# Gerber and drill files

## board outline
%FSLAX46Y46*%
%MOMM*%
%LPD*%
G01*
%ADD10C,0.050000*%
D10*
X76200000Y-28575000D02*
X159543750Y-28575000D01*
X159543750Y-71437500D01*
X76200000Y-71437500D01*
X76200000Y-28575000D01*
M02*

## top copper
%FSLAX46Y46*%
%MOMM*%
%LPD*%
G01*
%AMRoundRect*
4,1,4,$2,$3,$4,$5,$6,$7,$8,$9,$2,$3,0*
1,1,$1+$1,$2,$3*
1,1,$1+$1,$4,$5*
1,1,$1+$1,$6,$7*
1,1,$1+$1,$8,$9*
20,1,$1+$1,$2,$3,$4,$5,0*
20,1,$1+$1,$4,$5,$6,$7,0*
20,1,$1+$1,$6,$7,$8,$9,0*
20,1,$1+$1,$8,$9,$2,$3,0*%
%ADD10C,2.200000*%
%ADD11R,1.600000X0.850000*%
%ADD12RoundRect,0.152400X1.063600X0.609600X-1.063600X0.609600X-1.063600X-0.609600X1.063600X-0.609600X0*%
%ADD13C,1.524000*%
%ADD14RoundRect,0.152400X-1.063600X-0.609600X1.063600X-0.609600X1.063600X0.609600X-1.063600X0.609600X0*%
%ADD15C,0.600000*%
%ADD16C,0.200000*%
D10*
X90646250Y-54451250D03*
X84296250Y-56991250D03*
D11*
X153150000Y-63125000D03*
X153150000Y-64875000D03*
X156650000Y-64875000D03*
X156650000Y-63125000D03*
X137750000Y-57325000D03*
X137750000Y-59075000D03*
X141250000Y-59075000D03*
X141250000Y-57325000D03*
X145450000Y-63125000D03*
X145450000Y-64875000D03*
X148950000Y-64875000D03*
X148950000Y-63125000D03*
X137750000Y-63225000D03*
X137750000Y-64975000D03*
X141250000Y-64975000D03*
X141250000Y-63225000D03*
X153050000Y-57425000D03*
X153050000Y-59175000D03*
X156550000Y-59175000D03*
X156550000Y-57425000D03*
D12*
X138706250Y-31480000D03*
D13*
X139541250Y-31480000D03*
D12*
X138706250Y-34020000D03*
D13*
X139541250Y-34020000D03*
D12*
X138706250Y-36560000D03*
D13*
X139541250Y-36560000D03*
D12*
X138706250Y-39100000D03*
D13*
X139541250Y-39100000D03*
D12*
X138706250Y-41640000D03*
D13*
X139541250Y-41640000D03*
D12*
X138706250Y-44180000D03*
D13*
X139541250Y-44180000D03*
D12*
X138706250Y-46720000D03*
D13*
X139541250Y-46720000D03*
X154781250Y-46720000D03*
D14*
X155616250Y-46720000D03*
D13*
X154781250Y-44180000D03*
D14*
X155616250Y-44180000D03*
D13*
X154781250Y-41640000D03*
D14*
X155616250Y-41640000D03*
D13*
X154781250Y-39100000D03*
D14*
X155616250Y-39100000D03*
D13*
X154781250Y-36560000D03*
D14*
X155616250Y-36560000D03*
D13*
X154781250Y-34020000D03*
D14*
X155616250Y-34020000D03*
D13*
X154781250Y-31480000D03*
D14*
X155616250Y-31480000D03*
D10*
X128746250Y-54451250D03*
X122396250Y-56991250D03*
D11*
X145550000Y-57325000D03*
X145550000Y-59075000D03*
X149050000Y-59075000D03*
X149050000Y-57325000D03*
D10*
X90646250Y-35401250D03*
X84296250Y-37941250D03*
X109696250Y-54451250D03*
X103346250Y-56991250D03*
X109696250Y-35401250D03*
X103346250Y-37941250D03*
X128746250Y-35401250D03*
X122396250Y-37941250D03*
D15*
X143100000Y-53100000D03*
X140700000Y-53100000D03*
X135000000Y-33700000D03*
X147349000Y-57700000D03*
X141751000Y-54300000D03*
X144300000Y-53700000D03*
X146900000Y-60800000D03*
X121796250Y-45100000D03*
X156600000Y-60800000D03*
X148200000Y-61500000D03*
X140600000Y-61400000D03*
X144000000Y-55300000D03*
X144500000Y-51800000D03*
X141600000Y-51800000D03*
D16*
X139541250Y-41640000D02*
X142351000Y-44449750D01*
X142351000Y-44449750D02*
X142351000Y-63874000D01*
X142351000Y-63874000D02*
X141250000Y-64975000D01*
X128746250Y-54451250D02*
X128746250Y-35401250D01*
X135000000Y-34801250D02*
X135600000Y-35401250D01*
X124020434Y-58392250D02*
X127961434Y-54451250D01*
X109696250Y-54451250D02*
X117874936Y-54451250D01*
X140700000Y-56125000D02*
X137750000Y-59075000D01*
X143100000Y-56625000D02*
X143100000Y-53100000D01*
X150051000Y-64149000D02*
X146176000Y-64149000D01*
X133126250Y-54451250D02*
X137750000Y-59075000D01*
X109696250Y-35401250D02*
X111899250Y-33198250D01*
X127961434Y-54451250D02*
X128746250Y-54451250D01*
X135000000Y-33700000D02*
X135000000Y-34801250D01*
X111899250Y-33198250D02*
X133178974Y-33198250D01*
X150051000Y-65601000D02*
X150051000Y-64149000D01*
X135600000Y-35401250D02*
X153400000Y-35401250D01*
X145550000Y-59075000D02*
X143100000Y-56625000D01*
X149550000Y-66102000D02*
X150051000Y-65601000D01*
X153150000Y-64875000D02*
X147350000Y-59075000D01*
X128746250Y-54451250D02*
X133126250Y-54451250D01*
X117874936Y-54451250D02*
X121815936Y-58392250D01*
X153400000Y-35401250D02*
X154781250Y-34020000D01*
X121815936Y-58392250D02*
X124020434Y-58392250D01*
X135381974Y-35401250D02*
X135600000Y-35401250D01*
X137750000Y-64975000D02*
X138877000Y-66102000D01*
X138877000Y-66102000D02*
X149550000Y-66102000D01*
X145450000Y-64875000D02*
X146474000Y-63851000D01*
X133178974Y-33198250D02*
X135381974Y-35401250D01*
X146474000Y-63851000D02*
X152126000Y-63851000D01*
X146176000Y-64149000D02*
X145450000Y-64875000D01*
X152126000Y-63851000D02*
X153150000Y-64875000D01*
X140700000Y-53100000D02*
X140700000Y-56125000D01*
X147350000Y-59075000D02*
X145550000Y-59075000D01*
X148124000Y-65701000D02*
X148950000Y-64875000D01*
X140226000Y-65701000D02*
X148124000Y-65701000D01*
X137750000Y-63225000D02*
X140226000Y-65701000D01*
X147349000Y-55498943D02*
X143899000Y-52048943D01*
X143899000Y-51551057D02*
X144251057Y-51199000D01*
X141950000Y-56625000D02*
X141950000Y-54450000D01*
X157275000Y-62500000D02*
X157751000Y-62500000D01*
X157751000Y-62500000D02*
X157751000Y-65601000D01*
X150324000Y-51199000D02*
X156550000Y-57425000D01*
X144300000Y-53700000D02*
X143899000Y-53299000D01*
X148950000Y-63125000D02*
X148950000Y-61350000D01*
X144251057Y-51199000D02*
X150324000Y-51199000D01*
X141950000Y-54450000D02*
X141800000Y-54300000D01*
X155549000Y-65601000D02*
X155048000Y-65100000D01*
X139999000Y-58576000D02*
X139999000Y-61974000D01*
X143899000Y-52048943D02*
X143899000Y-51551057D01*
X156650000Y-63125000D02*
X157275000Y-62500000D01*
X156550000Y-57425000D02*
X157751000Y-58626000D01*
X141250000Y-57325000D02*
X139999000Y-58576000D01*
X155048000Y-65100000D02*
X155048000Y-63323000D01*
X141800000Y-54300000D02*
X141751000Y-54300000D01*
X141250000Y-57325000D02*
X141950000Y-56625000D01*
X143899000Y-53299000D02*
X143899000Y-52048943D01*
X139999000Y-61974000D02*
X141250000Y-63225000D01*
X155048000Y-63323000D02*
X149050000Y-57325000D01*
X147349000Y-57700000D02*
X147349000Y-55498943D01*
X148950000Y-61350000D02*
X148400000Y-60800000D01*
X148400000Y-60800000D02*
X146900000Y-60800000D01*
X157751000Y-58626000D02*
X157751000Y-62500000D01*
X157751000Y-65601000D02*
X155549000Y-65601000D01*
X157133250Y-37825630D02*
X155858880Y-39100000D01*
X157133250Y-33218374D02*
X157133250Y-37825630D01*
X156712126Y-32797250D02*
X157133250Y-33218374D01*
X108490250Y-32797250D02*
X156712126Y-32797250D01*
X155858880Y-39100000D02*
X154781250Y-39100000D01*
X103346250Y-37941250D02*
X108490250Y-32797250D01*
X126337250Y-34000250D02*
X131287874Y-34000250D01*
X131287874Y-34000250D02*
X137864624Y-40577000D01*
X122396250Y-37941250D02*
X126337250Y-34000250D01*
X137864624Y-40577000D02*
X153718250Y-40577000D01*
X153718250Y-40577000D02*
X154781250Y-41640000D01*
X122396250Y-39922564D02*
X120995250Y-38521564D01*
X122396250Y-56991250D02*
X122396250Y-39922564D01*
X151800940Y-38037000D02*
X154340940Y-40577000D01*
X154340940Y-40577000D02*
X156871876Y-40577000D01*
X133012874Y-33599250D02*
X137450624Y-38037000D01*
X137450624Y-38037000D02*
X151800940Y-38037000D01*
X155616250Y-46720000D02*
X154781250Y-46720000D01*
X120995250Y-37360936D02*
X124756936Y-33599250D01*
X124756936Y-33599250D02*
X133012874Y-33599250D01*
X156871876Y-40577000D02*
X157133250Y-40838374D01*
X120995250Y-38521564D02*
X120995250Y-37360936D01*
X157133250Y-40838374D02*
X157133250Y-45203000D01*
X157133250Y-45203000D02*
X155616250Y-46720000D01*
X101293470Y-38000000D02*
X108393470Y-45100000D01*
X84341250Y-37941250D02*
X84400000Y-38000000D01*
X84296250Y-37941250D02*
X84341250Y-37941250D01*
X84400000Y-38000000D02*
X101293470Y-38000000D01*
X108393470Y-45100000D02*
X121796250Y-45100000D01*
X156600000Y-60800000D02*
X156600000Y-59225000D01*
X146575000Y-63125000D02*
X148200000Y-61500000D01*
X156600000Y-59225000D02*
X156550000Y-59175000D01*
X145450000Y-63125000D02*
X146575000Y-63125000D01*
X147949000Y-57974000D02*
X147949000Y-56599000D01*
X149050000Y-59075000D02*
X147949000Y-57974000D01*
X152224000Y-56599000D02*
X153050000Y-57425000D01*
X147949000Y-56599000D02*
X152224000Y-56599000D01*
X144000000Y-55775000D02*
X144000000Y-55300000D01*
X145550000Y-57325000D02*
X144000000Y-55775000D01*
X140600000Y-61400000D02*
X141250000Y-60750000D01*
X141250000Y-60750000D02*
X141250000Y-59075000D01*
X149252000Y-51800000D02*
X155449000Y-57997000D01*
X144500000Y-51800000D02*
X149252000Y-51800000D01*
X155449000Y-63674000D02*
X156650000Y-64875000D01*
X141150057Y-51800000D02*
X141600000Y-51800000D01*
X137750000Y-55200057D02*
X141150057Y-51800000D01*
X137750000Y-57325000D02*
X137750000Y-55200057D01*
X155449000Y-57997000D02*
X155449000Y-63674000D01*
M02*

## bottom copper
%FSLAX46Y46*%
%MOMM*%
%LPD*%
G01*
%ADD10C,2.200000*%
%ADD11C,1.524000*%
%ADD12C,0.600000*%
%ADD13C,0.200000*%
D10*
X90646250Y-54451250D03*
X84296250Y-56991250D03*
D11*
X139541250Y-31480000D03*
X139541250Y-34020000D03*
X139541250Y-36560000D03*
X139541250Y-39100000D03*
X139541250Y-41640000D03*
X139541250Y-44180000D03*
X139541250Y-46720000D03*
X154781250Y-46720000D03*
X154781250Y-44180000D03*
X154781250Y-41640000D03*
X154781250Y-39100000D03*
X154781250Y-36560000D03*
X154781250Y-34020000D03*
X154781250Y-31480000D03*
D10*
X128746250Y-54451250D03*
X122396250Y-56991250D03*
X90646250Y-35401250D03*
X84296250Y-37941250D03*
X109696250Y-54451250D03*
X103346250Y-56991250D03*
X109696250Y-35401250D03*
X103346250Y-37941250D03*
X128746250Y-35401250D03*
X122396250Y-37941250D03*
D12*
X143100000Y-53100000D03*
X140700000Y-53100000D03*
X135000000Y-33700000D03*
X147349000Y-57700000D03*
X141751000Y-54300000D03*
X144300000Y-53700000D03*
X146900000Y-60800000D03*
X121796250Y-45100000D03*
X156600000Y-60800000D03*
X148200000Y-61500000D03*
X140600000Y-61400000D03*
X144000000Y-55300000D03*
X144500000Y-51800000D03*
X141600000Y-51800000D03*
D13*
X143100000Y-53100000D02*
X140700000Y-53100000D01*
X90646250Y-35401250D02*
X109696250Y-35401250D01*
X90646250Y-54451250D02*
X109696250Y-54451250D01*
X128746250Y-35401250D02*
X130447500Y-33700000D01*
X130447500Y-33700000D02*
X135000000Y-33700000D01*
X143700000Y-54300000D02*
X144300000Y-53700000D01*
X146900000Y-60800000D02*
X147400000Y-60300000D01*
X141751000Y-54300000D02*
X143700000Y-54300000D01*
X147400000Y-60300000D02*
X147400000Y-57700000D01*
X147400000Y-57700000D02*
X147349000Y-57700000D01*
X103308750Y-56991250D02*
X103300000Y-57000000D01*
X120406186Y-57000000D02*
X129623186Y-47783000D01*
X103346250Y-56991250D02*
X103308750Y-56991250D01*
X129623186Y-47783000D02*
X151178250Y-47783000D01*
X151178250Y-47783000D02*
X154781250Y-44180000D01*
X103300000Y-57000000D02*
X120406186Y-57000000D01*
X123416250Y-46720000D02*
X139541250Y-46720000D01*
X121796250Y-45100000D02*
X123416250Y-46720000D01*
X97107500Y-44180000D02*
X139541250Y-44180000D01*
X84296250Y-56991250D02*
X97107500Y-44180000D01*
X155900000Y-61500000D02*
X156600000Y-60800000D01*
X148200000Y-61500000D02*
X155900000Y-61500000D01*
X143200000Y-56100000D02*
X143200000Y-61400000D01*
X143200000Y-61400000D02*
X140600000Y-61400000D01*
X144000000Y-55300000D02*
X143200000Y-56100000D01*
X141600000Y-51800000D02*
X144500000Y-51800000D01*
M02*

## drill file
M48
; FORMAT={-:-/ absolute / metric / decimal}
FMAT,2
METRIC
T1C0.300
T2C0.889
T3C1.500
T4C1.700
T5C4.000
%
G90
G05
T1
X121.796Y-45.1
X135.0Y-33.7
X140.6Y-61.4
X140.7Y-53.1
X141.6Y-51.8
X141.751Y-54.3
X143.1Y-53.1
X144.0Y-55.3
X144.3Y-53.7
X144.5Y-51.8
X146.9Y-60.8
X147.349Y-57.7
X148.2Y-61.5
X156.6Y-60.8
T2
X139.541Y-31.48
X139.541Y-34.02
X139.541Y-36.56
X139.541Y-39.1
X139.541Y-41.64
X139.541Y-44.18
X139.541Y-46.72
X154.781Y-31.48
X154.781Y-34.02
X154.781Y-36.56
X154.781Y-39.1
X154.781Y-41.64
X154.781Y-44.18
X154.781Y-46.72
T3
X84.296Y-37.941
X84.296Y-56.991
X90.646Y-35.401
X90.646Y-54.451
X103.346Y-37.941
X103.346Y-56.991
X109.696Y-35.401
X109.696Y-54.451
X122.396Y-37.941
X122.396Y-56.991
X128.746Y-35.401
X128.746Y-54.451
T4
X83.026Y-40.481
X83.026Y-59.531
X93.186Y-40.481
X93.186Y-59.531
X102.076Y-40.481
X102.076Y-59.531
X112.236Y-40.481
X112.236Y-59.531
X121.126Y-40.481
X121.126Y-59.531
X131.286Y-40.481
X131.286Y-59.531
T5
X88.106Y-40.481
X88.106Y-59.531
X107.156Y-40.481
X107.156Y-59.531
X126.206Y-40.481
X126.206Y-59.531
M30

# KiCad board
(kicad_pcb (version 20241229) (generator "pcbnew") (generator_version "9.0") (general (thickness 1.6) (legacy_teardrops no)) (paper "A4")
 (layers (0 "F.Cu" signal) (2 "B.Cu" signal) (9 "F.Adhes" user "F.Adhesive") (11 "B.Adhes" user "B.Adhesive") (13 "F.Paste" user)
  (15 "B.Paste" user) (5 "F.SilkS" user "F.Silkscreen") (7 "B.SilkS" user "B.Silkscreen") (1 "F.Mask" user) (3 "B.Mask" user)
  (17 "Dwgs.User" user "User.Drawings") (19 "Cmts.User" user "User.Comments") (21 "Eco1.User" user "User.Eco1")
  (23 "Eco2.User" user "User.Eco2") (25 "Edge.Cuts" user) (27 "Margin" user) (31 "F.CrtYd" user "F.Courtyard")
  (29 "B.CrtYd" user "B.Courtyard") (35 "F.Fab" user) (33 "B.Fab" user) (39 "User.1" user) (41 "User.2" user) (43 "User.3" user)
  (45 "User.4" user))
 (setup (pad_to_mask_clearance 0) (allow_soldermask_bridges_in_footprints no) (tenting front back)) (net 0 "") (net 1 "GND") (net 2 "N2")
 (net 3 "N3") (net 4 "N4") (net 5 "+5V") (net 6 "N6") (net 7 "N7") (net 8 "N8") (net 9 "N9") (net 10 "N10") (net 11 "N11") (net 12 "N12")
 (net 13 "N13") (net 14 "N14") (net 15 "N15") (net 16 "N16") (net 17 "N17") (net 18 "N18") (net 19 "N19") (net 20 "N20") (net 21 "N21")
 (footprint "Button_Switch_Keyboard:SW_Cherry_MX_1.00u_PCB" (layer "F.Cu") (at 90.64625 54.45125)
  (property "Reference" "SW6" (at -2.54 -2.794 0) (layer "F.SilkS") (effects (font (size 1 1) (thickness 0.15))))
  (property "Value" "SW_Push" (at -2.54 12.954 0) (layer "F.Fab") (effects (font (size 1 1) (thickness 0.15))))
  (pad "" np_thru_hole circle (at -7.62 5.08) (size 1.7 1.7) (drill 1.7) (layers "*.Cu" "*.Mask"))
  (pad "" np_thru_hole circle (at -2.54 5.08) (size 4 4) (drill 4) (layers "*.Cu" "*.Mask"))
  (pad "" np_thru_hole circle (at 2.54 5.08) (size 1.7 1.7) (drill 1.7) (layers "*.Cu" "*.Mask"))
  (pad "1" thru_hole circle (at 0 0) (size 2.2 2.2) (drill 1.5) (layers "*.Cu" "*.Mask") (remove_unused_layers no) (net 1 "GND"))
  (pad "2" thru_hole circle (at -6.35 2.54) (size 2.2 2.2) (drill 1.5) (layers "*.Cu" "*.Mask") (remove_unused_layers no) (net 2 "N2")))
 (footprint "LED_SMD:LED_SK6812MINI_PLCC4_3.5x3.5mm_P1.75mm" (layer "F.Cu") (at 154.9 64)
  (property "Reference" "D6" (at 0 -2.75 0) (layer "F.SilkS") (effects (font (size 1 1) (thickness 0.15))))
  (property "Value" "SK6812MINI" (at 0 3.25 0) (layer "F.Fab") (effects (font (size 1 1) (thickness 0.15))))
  (pad "1" smd rect (at -1.75 -0.875) (size 1.6 0.85) (layers "F.Cu" "F.Mask" "F.Paste") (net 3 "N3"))
  (pad "2" smd rect (at -1.75 0.875) (size 1.6 0.85) (layers "F.Cu" "F.Mask" "F.Paste") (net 1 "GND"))
  (pad "3" smd rect (at 1.75 0.875) (size 1.6 0.85) (layers "F.Cu" "F.Mask" "F.Paste") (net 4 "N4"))
  (pad "4" smd rect (at 1.75 -0.875) (size 1.6 0.85) (layers "F.Cu" "F.Mask" "F.Paste") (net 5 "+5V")))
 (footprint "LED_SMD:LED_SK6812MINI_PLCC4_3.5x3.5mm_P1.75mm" (layer "F.Cu") (at 139.5 58.2)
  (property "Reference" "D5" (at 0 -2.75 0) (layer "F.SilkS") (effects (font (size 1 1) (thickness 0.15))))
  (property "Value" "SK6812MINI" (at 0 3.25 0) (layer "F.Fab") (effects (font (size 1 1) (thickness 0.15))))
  (pad "1" smd rect (at -1.75 -0.875) (size 1.6 0.85) (layers "F.Cu" "F.Mask" "F.Paste") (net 4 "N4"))
  (pad "2" smd rect (at -1.75 0.875) (size 1.6 0.85) (layers "F.Cu" "F.Mask" "F.Paste") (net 1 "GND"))
  (pad "3" smd rect (at 1.75 0.875) (size 1.6 0.85) (layers "F.Cu" "F.Mask" "F.Paste") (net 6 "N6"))
  (pad "4" smd rect (at 1.75 -0.875) (size 1.6 0.85) (layers "F.Cu" "F.Mask" "F.Paste") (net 5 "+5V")))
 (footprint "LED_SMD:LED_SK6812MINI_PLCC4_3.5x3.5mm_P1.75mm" (layer "F.Cu") (at 147.2 64)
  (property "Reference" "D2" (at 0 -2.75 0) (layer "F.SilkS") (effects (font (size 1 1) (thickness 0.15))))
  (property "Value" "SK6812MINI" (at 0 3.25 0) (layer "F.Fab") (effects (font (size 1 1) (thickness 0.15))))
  (pad "1" smd rect (at -1.75 -0.875) (size 1.6 0.85) (layers "F.Cu" "F.Mask" "F.Paste") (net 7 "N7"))
  (pad "2" smd rect (at -1.75 0.875) (size 1.6 0.85) (layers "F.Cu" "F.Mask" "F.Paste") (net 1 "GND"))
  (pad "3" smd rect (at 1.75 0.875) (size 1.6 0.85) (layers "F.Cu" "F.Mask" "F.Paste") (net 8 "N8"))
  (pad "4" smd rect (at 1.75 -0.875) (size 1.6 0.85) (layers "F.Cu" "F.Mask" "F.Paste") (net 5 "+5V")))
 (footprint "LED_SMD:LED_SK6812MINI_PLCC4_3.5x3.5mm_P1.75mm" (layer "F.Cu") (at 139.5 64.1)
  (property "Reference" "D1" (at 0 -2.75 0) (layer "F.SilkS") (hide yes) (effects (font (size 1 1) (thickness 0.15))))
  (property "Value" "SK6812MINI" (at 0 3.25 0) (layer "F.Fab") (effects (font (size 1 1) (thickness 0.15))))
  (pad "1" smd rect (at -1.75 -0.875) (size 1.6 0.85) (layers "F.Cu" "F.Mask" "F.Paste") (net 8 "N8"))
  (pad "2" smd rect (at -1.75 0.875) (size 1.6 0.85) (layers "F.Cu" "F.Mask" "F.Paste") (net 1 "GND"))
  (pad "3" smd rect (at 1.75 0.875) (size 1.6 0.85) (layers "F.Cu" "F.Mask" "F.Paste") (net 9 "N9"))
  (pad "4" smd rect (at 1.75 -0.875) (size 1.6 0.85) (layers "F.Cu" "F.Mask" "F.Paste") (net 5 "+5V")))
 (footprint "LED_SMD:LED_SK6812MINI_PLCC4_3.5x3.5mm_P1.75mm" (layer "F.Cu") (at 154.8 58.3)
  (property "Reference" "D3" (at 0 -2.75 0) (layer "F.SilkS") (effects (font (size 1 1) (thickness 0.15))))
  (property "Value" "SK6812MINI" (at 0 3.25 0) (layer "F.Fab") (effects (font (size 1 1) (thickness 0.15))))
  (pad "1" smd rect (at -1.75 -0.875) (size 1.6 0.85) (layers "F.Cu" "F.Mask" "F.Paste") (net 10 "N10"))
  (pad "2" smd rect (at -1.75 0.875) (size 1.6 0.85) (layers "F.Cu" "F.Mask" "F.Paste") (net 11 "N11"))
  (pad "3" smd rect (at 1.75 0.875) (size 1.6 0.85) (layers "F.Cu" "F.Mask" "F.Paste") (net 7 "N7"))
  (pad "4" smd rect (at 1.75 -0.875) (size 1.6 0.85) (layers "F.Cu" "F.Mask" "F.Paste") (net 5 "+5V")))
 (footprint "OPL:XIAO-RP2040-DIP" (layer "F.Cu") (at 147.16125 39.1)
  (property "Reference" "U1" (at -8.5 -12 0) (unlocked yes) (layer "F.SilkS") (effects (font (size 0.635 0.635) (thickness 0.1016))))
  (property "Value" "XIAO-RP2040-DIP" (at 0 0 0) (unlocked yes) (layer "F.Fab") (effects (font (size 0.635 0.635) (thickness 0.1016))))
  (pad "1" smd roundrect (at -8.455 -7.62 180) (size 2.432 1.524) (layers "F.Cu" "F.Mask") (roundrect_rratio 0.1) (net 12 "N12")
   (thermal_bridge_angle 45))
  (pad "1" thru_hole circle (at -7.62 -7.62 180) (size 1.524 1.524) (drill 0.889) (layers "*.Cu" "*.Mask") (remove_unused_layers no)
   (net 12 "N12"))
  (pad "2" smd roundrect (at -8.455 -5.08 180) (size 2.432 1.524) (layers "F.Cu" "F.Mask") (roundrect_rratio 0.1) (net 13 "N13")
   (thermal_bridge_angle 45))
  (pad "2" thru_hole circle (at -7.62 -5.08 180) (size 1.524 1.524) (drill 0.889) (layers "*.Cu" "*.Mask") (remove_unused_layers no)
   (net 13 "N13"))
  (pad "3" smd roundrect (at -8.455 -2.54 180) (size 2.432 1.524) (layers "F.Cu" "F.Mask") (roundrect_rratio 0.1) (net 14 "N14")
   (thermal_bridge_angle 45))
  (pad "3" thru_hole circle (at -7.62 -2.54 180) (size 1.524 1.524) (drill 0.889) (layers "*.Cu" "*.Mask") (remove_unused_layers no)
   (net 14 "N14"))
  (pad "4" smd roundrect (at -8.455 0 180) (size 2.432 1.524) (layers "F.Cu" "F.Mask") (roundrect_rratio 0.1) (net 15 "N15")
   (thermal_bridge_angle 45))
  (pad "4" thru_hole circle (at -7.62 0 180) (size 1.524 1.524) (drill 0.889) (layers "*.Cu" "*.Mask") (remove_unused_layers no)
   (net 15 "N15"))
  (pad "5" smd roundrect (at -8.455 2.54 180) (size 2.432 1.524) (layers "F.Cu" "F.Mask") (roundrect_rratio 0.1) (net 9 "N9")
   (thermal_bridge_angle 45))
  (pad "5" thru_hole circle (at -7.62 2.54 180) (size 1.524 1.524) (drill 0.889) (layers "*.Cu" "*.Mask") (remove_unused_layers no)
   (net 9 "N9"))
  (pad "6" smd roundrect (at -8.455 5.08 180) (size 2.432 1.524) (layers "F.Cu" "F.Mask") (roundrect_rratio 0.1) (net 2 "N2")
   (thermal_bridge_angle 45))
  (pad "6" thru_hole circle (at -7.62 5.08 180) (size 1.524 1.524) (drill 0.889) (layers "*.Cu" "*.Mask") (remove_unused_layers no)
   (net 2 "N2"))
  (pad "7" smd roundrect (at -8.455 7.62 180) (size 2.432 1.524) (layers "F.Cu" "F.Mask") (roundrect_rratio 0.1) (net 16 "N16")
   (thermal_bridge_angle 45))
  (pad "7" thru_hole circle (at -7.62 7.62 180) (size 1.524 1.524) (drill 0.889) (layers "*.Cu" "*.Mask") (remove_unused_layers no)
   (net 16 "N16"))
  (pad "8" thru_hole circle (at 7.62 7.62) (size 1.524 1.524) (drill 0.889) (layers "*.Cu" "*.Mask") (remove_unused_layers no)
   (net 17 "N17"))
  (pad "8" smd roundrect (at 8.455 7.62) (size 2.432 1.524) (layers "F.Cu" "F.Mask") (roundrect_rratio 0.1) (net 17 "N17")
   (thermal_bridge_angle 45))
  (pad "9" thru_hole circle (at 7.62 5.08) (size 1.524 1.524) (drill 0.889) (layers "*.Cu" "*.Mask") (remove_unused_layers no)
   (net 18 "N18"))
  (pad "9" smd roundrect (at 8.455 5.08) (size 2.432 1.524) (layers "F.Cu" "F.Mask") (roundrect_rratio 0.1) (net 18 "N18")
   (thermal_bridge_angle 45))
  (pad "10" thru_hole circle (at 7.62 2.54) (size 1.524 1.524) (drill 0.889) (layers "*.Cu" "*.Mask") (remove_unused_layers no)
   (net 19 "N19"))
  (pad "10" smd roundrect (at 8.455 2.54) (size 2.432 1.524) (layers "F.Cu" "F.Mask") (roundrect_rratio 0.1) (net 19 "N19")
   (thermal_bridge_angle 45))
  (pad "11" thru_hole circle (at 7.62 0) (size 1.524 1.524) (drill 0.889) (layers "*.Cu" "*.Mask") (remove_unused_layers no) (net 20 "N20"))
  (pad "11" smd roundrect (at 8.455 0) (size 2.432 1.524) (layers "F.Cu" "F.Mask") (roundrect_rratio 0.1) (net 20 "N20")
   (thermal_bridge_angle 45))
  (pad "12" thru_hole circle (at 7.62 -2.54) (size 1.524 1.524) (drill 0.889) (layers "*.Cu" "*.Mask") (remove_unused_layers no)
   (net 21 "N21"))
  (pad "12" smd roundrect (at 8.455 -2.54) (size 2.432 1.524) (layers "F.Cu" "F.Mask") (roundrect_rratio 0.1) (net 21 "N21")
   (thermal_bridge_angle 45))
  (pad "13" thru_hole circle (at 7.62 -5.08) (size 1.524 1.524) (drill 0.889) (layers "*.Cu" "*.Mask") (remove_unused_layers no)
   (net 1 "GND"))
  (pad "13" smd roundrect (at 8.455 -5.08) (size 2.432 1.524) (layers "F.Cu" "F.Mask") (roundrect_rratio 0.1) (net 1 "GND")
   (thermal_bridge_angle 45))
  (pad "14" thru_hole circle (at 7.62 -7.62) (size 1.524 1.524) (drill 0.889) (layers "*.Cu" "*.Mask") (remove_unused_layers no)
   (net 5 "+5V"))
  (pad "14" smd roundrect (at 8.455 -7.62) (size 2.432 1.524) (layers "F.Cu" "F.Mask") (roundrect_rratio 0.1) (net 5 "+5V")
   (thermal_bridge_angle 45)))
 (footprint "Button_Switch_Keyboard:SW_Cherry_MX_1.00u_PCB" (layer "F.Cu") (at 128.74625 54.45125)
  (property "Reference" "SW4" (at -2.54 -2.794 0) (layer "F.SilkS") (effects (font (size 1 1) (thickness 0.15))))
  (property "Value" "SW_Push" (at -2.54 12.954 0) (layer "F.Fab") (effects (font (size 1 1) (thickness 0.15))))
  (pad "" np_thru_hole circle (at -7.62 5.08) (size 1.7 1.7) (drill 1.7) (layers "*.Cu" "*.Mask"))
  (pad "" np_thru_hole circle (at -2.54 5.08) (size 4 4) (drill 4) (layers "*.Cu" "*.Mask"))
  (pad "" np_thru_hole circle (at 2.54 5.08) (size 1.7 1.7) (drill 1.7) (layers "*.Cu" "*.Mask"))
  (pad "1" thru_hole circle (at 0 0) (size 2.2 2.2) (drill 1.5) (layers "*.Cu" "*.Mask") (remove_unused_layers no) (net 1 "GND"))
  (pad "2" thru_hole circle (at -6.35 2.54) (size 2.2 2.2) (drill 1.5) (layers "*.Cu" "*.Mask") (remove_unused_layers no) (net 17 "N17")))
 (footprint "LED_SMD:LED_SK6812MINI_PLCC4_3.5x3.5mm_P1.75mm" (layer "F.Cu") (at 147.3 58.2)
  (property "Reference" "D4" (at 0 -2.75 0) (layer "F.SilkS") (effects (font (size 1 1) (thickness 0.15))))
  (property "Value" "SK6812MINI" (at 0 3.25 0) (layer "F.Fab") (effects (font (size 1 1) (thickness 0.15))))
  (pad "1" smd rect (at -1.75 -0.875) (size 1.6 0.85) (layers "F.Cu" "F.Mask" "F.Paste") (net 6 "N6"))
  (pad "2" smd rect (at -1.75 0.875) (size 1.6 0.85) (layers "F.Cu" "F.Mask" "F.Paste") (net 1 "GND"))
  (pad "3" smd rect (at 1.75 0.875) (size 1.6 0.85) (layers "F.Cu" "F.Mask" "F.Paste") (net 10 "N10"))
  (pad "4" smd rect (at 1.75 -0.875) (size 1.6 0.85) (layers "F.Cu" "F.Mask" "F.Paste") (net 5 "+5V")))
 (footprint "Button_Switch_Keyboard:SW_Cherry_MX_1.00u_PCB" (layer "F.Cu") (at 90.64625 35.40125)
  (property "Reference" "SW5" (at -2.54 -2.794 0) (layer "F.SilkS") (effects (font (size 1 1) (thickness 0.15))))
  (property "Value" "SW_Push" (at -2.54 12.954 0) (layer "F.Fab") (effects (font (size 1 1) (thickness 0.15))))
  (pad "" np_thru_hole circle (at -7.62 5.08) (size 1.7 1.7) (drill 1.7) (layers "*.Cu" "*.Mask"))
  (pad "" np_thru_hole circle (at -2.54 5.08) (size 4 4) (drill 4) (layers "*.Cu" "*.Mask"))
  (pad "" np_thru_hole circle (at 2.54 5.08) (size 1.7 1.7) (drill 1.7) (layers "*.Cu" "*.Mask"))
  (pad "1" thru_hole circle (at 0 0) (size 2.2 2.2) (drill 1.5) (layers "*.Cu" "*.Mask") (remove_unused_layers no) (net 1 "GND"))
  (pad "2" thru_hole circle (at -6.35 2.54) (size 2.2 2.2) (drill 1.5) (layers "*.Cu" "*.Mask") (remove_unused_layers no) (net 16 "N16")))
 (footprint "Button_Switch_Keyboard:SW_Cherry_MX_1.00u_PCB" (layer "F.Cu") (at 109.69625 54.45125)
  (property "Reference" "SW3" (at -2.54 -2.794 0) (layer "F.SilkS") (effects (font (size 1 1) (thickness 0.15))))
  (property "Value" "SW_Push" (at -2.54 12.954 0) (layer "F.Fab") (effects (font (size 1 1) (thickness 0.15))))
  (pad "" np_thru_hole circle (at -7.62 5.08) (size 1.7 1.7) (drill 1.7) (layers "*.Cu" "*.Mask"))
  (pad "" np_thru_hole circle (at -2.54 5.08) (size 4 4) (drill 4) (layers "*.Cu" "*.Mask"))
  (pad "" np_thru_hole circle (at 2.54 5.08) (size 1.7 1.7) (drill 1.7) (layers "*.Cu" "*.Mask"))
  (pad "1" thru_hole circle (at 0 0) (size 2.2 2.2) (drill 1.5) (layers "*.Cu" "*.Mask") (remove_unused_layers no) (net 1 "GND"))
  (pad "2" thru_hole circle (at -6.35 2.54) (size 2.2 2.2) (drill 1.5) (layers "*.Cu" "*.Mask") (remove_unused_layers no) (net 18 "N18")))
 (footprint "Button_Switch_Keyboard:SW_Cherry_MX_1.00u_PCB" (layer "F.Cu") (at 109.69625 35.40125)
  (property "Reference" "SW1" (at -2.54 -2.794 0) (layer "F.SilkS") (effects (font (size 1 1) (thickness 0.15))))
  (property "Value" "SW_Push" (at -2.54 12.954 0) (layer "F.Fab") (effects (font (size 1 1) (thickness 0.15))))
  (pad "" np_thru_hole circle (at -7.62 5.08) (size 1.7 1.7) (drill 1.7) (layers "*.Cu" "*.Mask"))
  (pad "" np_thru_hole circle (at -2.54 5.08) (size 4 4) (drill 4) (layers "*.Cu" "*.Mask"))
  (pad "" np_thru_hole circle (at 2.54 5.08) (size 1.7 1.7) (drill 1.7) (layers "*.Cu" "*.Mask"))
  (pad "1" thru_hole circle (at 0 0) (size 2.2 2.2) (drill 1.5) (layers "*.Cu" "*.Mask") (remove_unused_layers no) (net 1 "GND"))
  (pad "2" thru_hole circle (at -6.35 2.54) (size 2.2 2.2) (drill 1.5) (layers "*.Cu" "*.Mask") (remove_unused_layers no) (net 20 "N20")))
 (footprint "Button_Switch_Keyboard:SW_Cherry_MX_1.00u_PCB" (layer "F.Cu") (at 128.74625 35.40125)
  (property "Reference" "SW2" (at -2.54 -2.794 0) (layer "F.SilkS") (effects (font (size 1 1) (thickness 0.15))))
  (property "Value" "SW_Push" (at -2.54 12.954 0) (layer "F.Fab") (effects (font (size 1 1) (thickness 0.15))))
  (pad "" np_thru_hole circle (at -7.62 5.08) (size 1.7 1.7) (drill 1.7) (layers "*.Cu" "*.Mask"))
  (pad "" np_thru_hole circle (at -2.54 5.08) (size 4 4) (drill 4) (layers "*.Cu" "*.Mask"))
  (pad "" np_thru_hole circle (at 2.54 5.08) (size 1.7 1.7) (drill 1.7) (layers "*.Cu" "*.Mask"))
  (pad "1" thru_hole circle (at 0 0) (size 2.2 2.2) (drill 1.5) (layers "*.Cu" "*.Mask") (remove_unused_layers no) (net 1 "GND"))
  (pad "2" thru_hole circle (at -6.35 2.54) (size 2.2 2.2) (drill 1.5) (layers "*.Cu" "*.Mask") (remove_unused_layers no) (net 19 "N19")))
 (gr_rect (start 76.2 28.575) (end 159.54375 71.4375) (stroke (width 0.05) (type default)) (fill no) (layer "Edge.Cuts"))
 (segment (start 139.54125 41.64) (end 142.351 44.44975) (width 0.2) (layer "F.Cu") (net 9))
 (segment (start 142.351 44.44975) (end 142.351 63.874) (width 0.2) (layer "F.Cu") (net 9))
 (segment (start 142.351 63.874) (end 141.25 64.975) (width 0.2) (layer "F.Cu") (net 9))
 (segment (start 128.74625 54.45125) (end 128.74625 35.40125) (width 0.2) (layer "F.Cu") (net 1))
 (segment (start 135 34.80125) (end 135.6 35.40125) (width 0.2) (layer "F.Cu") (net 1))
 (segment (start 124.020434 58.39225) (end 127.961434 54.45125) (width 0.2) (layer "F.Cu") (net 1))
 (segment (start 109.69625 54.45125) (end 117.874936 54.45125) (width 0.2) (layer "F.Cu") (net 1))
 (segment (start 140.7 56.125) (end 137.75 59.075) (width 0.2) (layer "F.Cu") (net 1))
 (segment (start 143.1 56.625) (end 143.1 53.1) (width 0.2) (layer "F.Cu") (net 1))
 (segment (start 150.051 64.149) (end 146.176 64.149) (width 0.2) (layer "F.Cu") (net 1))
 (segment (start 133.12625 54.45125) (end 137.75 59.075) (width 0.2) (layer "F.Cu") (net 1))
 (segment (start 109.69625 35.40125) (end 111.89925 33.19825) (width 0.2) (layer "F.Cu") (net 1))
 (segment (start 127.961434 54.45125) (end 128.74625 54.45125) (width 0.2) (layer "F.Cu") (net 1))
 (segment (start 135 33.7) (end 135 34.80125) (width 0.2) (layer "F.Cu") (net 1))
 (segment (start 111.89925 33.19825) (end 133.178974 33.19825) (width 0.2) (layer "F.Cu") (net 1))
 (segment (start 150.051 65.601) (end 150.051 64.149) (width 0.2) (layer "F.Cu") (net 1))
 (segment (start 135.6 35.40125) (end 153.4 35.40125) (width 0.2) (layer "F.Cu") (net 1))
 (segment (start 145.55 59.075) (end 143.1 56.625) (width 0.2) (layer "F.Cu") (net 1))
 (segment (start 149.55 66.102) (end 150.051 65.601) (width 0.2) (layer "F.Cu") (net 1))
 (segment (start 153.15 64.875) (end 147.35 59.075) (width 0.2) (layer "F.Cu") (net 1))
 (segment (start 128.74625 54.45125) (end 133.12625 54.45125) (width 0.2) (layer "F.Cu") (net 1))
 (segment (start 117.874936 54.45125) (end 121.815936 58.39225) (width 0.2) (layer "F.Cu") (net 1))
 (segment (start 153.4 35.40125) (end 154.78125 34.02) (width 0.2) (layer "F.Cu") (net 1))
 (segment (start 121.815936 58.39225) (end 124.020434 58.39225) (width 0.2) (layer "F.Cu") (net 1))
 (segment (start 135.381974 35.40125) (end 135.6 35.40125) (width 0.2) (layer "F.Cu") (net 1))
 (segment (start 137.75 64.975) (end 138.877 66.102) (width 0.2) (layer "F.Cu") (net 1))
 (segment (start 138.877 66.102) (end 149.55 66.102) (width 0.2) (layer "F.Cu") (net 1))
 (segment (start 145.45 64.875) (end 146.474 63.851) (width 0.2) (layer "F.Cu") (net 1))
 (segment (start 133.178974 33.19825) (end 135.381974 35.40125) (width 0.2) (layer "F.Cu") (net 1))
 (segment (start 146.474 63.851) (end 152.126 63.851) (width 0.2) (layer "F.Cu") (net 1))
 (segment (start 146.176 64.149) (end 145.45 64.875) (width 0.2) (layer "F.Cu") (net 1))
 (segment (start 152.126 63.851) (end 153.15 64.875) (width 0.2) (layer "F.Cu") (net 1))
 (segment (start 140.7 53.1) (end 140.7 56.125) (width 0.2) (layer "F.Cu") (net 1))
 (segment (start 147.35 59.075) (end 145.55 59.075) (width 0.2) (layer "F.Cu") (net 1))
 (via (at 143.1 53.1) (size 0.6) (drill 0.3) (layers "F.Cu" "B.Cu") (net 1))
 (via (at 140.7 53.1) (size 0.6) (drill 0.3) (layers "F.Cu" "B.Cu") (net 1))
 (via (at 135 33.7) (size 0.6) (drill 0.3) (layers "F.Cu" "B.Cu") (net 1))
 (segment (start 143.1 53.1) (end 140.7 53.1) (width 0.2) (layer "B.Cu") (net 1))
 (segment (start 90.64625 35.40125) (end 109.69625 35.40125) (width 0.2) (layer "B.Cu") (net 1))
 (segment (start 90.64625 54.45125) (end 109.69625 54.45125) (width 0.2) (layer "B.Cu") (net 1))
 (segment (start 128.74625 35.40125) (end 130.4475 33.7) (width 0.2) (layer "B.Cu") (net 1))
 (segment (start 130.4475 33.7) (end 135 33.7) (width 0.2) (layer "B.Cu") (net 1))
 (segment (start 148.124 65.701) (end 148.95 64.875) (width 0.2) (layer "F.Cu") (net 8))
 (segment (start 140.226 65.701) (end 148.124 65.701) (width 0.2) (layer "F.Cu") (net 8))
 (segment (start 137.75 63.225) (end 140.226 65.701) (width 0.2) (layer "F.Cu") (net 8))
 (segment (start 147.349 55.498943) (end 143.899 52.048943) (width 0.2) (layer "F.Cu") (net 5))
 (segment (start 143.899 51.551057) (end 144.251057 51.199) (width 0.2) (layer "F.Cu") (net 5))
 (segment (start 141.95 56.625) (end 141.95 54.45) (width 0.2) (layer "F.Cu") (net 5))
 (segment (start 157.275 62.5) (end 157.751 62.5) (width 0.2) (layer "F.Cu") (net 5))
 (segment (start 157.751 62.5) (end 157.751 65.601) (width 0.2) (layer "F.Cu") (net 5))
 (segment (start 150.324 51.199) (end 156.55 57.425) (width 0.2) (layer "F.Cu") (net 5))
 (segment (start 144.3 53.7) (end 143.899 53.299) (width 0.2) (layer "F.Cu") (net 5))
 (segment (start 148.95 63.125) (end 148.95 61.35) (width 0.2) (layer "F.Cu") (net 5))
 (segment (start 144.251057 51.199) (end 150.324 51.199) (width 0.2) (layer "F.Cu") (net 5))
 (segment (start 141.95 54.45) (end 141.8 54.3) (width 0.2) (layer "F.Cu") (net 5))
 (segment (start 155.549 65.601) (end 155.048 65.1) (width 0.2) (layer "F.Cu") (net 5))
 (segment (start 139.999 58.576) (end 139.999 61.974) (width 0.2) (layer "F.Cu") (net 5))
 (segment (start 143.899 52.048943) (end 143.899 51.551057) (width 0.2) (layer "F.Cu") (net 5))
 (segment (start 156.65 63.125) (end 157.275 62.5) (width 0.2) (layer "F.Cu") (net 5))
 (segment (start 156.55 57.425) (end 157.751 58.626) (width 0.2) (layer "F.Cu") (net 5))
 (segment (start 141.25 57.325) (end 139.999 58.576) (width 0.2) (layer "F.Cu") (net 5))
 (segment (start 155.048 65.1) (end 155.048 63.323) (width 0.2) (layer "F.Cu") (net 5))
 (segment (start 141.8 54.3) (end 141.751 54.3) (width 0.2) (layer "F.Cu") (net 5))
 (segment (start 141.25 57.325) (end 141.95 56.625) (width 0.2) (layer "F.Cu") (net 5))
 (segment (start 143.899 53.299) (end 143.899 52.048943) (width 0.2) (layer "F.Cu") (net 5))
 (segment (start 139.999 61.974) (end 141.25 63.225) (width 0.2) (layer "F.Cu") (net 5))
 (segment (start 155.048 63.323) (end 149.05 57.325) (width 0.2) (layer "F.Cu") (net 5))
 (segment (start 147.349 57.7) (end 147.349 55.498943) (width 0.2) (layer "F.Cu") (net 5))
 (segment (start 148.95 61.35) (end 148.4 60.8) (width 0.2) (layer "F.Cu") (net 5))
 (segment (start 148.4 60.8) (end 146.9 60.8) (width 0.2) (layer "F.Cu") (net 5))
 (segment (start 157.751 58.626) (end 157.751 62.5) (width 0.2) (layer "F.Cu") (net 5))
 (segment (start 157.751 65.601) (end 155.549 65.601) (width 0.2) (layer "F.Cu") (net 5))
 (via (at 147.349 57.7) (size 0.6) (drill 0.3) (layers "F.Cu" "B.Cu") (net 5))
 (via (at 141.751 54.3) (size 0.6) (drill 0.3) (layers "F.Cu" "B.Cu") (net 5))
 (via (at 144.3 53.7) (size 0.6) (drill 0.3) (layers "F.Cu" "B.Cu") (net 5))
 (via (at 146.9 60.8) (size 0.6) (drill 0.3) (layers "F.Cu" "B.Cu") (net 5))
 (segment (start 143.7 54.3) (end 144.3 53.7) (width 0.2) (layer "B.Cu") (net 5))
 (segment (start 146.9 60.8) (end 147.4 60.3) (width 0.2) (layer "B.Cu") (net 5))
 (segment (start 141.751 54.3) (end 143.7 54.3) (width 0.2) (layer "B.Cu") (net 5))
 (segment (start 147.4 60.3) (end 147.4 57.7) (width 0.2) (layer "B.Cu") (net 5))
 (segment (start 147.4 57.7) (end 147.349 57.7) (width 0.2) (layer "B.Cu") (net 5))
 (segment (start 157.13325 37.82563) (end 155.85888 39.1) (width 0.2) (layer "F.Cu") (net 20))
 (segment (start 157.13325 33.218374) (end 157.13325 37.82563) (width 0.2) (layer "F.Cu") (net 20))
 (segment (start 156.712126 32.79725) (end 157.13325 33.218374) (width 0.2) (layer "F.Cu") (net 20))
 (segment (start 108.49025 32.79725) (end 156.712126 32.79725) (width 0.2) (layer "F.Cu") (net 20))
 (segment (start 155.85888 39.1) (end 154.78125 39.1) (width 0.2) (layer "F.Cu") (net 20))
 (segment (start 103.34625 37.94125) (end 108.49025 32.79725) (width 0.2) (layer "F.Cu") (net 20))
 (segment (start 126.33725 34.00025) (end 131.287874 34.00025) (width 0.2) (layer "F.Cu") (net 19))
 (segment (start 131.287874 34.00025) (end 137.864624 40.577) (width 0.2) (layer "F.Cu") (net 19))
 (segment (start 122.39625 37.94125) (end 126.33725 34.00025) (width 0.2) (layer "F.Cu") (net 19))
 (segment (start 137.864624 40.577) (end 153.71825 40.577) (width 0.2) (layer "F.Cu") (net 19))
 (segment (start 153.71825 40.577) (end 154.78125 41.64) (width 0.2) (layer "F.Cu") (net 19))
 (segment (start 103.30875 56.99125) (end 103.3 57) (width 0.2) (layer "B.Cu") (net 18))
 (segment (start 120.406186 57) (end 129.623186 47.783) (width 0.2) (layer "B.Cu") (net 18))
 (segment (start 103.34625 56.99125) (end 103.30875 56.99125) (width 0.2) (layer "B.Cu") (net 18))
 (segment (start 129.623186 47.783) (end 151.17825 47.783) (width 0.2) (layer "B.Cu") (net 18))
 (segment (start 151.17825 47.783) (end 154.78125 44.18) (width 0.2) (layer "B.Cu") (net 18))
 (segment (start 103.3 57) (end 120.406186 57) (width 0.2) (layer "B.Cu") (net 18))
 (segment (start 122.39625 39.922564) (end 120.99525 38.521564) (width 0.2) (layer "F.Cu") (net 17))
 (segment (start 122.39625 56.99125) (end 122.39625 39.922564) (width 0.2) (layer "F.Cu") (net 17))
 (segment (start 151.80094 38.037) (end 154.34094 40.577) (width 0.2) (layer "F.Cu") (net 17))
 (segment (start 154.34094 40.577) (end 156.871876 40.577) (width 0.2) (layer "F.Cu") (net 17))
 (segment (start 133.012874 33.59925) (end 137.450624 38.037) (width 0.2) (layer "F.Cu") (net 17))
 (segment (start 137.450624 38.037) (end 151.80094 38.037) (width 0.2) (layer "F.Cu") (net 17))
 (segment (start 155.61625 46.72) (end 154.78125 46.72) (width 0.2) (layer "F.Cu") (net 17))
 (segment (start 120.99525 37.360936) (end 124.756936 33.59925) (width 0.2) (layer "F.Cu") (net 17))
 (segment (start 124.756936 33.59925) (end 133.012874 33.59925) (width 0.2) (layer "F.Cu") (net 17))
 (segment (start 156.871876 40.577) (end 157.13325 40.838374) (width 0.2) (layer "F.Cu") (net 17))
 (segment (start 120.99525 38.521564) (end 120.99525 37.360936) (width 0.2) (layer "F.Cu") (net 17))
 (segment (start 157.13325 40.838374) (end 157.13325 45.203) (width 0.2) (layer "F.Cu") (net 17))
 (segment (start 157.13325 45.203) (end 155.61625 46.72) (width 0.2) (layer "F.Cu") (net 17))
 (segment (start 101.29347 38) (end 108.39347 45.1) (width 0.2) (layer "F.Cu") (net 16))
 (segment (start 84.34125 37.94125) (end 84.4 38) (width 0.2) (layer "F.Cu") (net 16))
 (segment (start 84.29625 37.94125) (end 84.34125 37.94125) (width 0.2) (layer "F.Cu") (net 16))
 (segment (start 84.4 38) (end 101.29347 38) (width 0.2) (layer "F.Cu") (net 16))
 (segment (start 108.39347 45.1) (end 121.79625 45.1) (width 0.2) (layer "F.Cu") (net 16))
 (via (at 121.79625 45.1) (size 0.6) (drill 0.3) (layers "F.Cu" "B.Cu") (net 16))
 (segment (start 123.41625 46.72) (end 139.54125 46.72) (width 0.2) (layer "B.Cu") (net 16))
 (segment (start 121.79625 45.1) (end 123.41625 46.72) (width 0.2) (layer "B.Cu") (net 16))
 (segment (start 97.1075 44.18) (end 139.54125 44.18) (width 0.2) (layer "B.Cu") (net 2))
 (segment (start 84.29625 56.99125) (end 97.1075 44.18) (width 0.2) (layer "B.Cu") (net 2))
 (segment (start 156.6 60.8) (end 156.6 59.225) (width 0.2) (layer "F.Cu") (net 7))
 (segment (start 146.575 63.125) (end 148.2 61.5) (width 0.2) (layer "F.Cu") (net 7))
 (segment (start 156.6 59.225) (end 156.55 59.175) (width 0.2) (layer "F.Cu") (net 7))
 (segment (start 145.45 63.125) (end 146.575 63.125) (width 0.2) (layer "F.Cu") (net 7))
 (via (at 156.6 60.8) (size 0.6) (drill 0.3) (layers "F.Cu" "B.Cu") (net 7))
 (via (at 148.2 61.5) (size 0.6) (drill 0.3) (layers "F.Cu" "B.Cu") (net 7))
 (segment (start 155.9 61.5) (end 156.6 60.8) (width 0.2) (layer "B.Cu") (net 7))
 (segment (start 148.2 61.5) (end 155.9 61.5) (width 0.2) (layer "B.Cu") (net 7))
 (segment (start 147.949 57.974) (end 147.949 56.599) (width 0.2) (layer "F.Cu") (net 10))
 (segment (start 149.05 59.075) (end 147.949 57.974) (width 0.2) (layer "F.Cu") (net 10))
 (segment (start 152.224 56.599) (end 153.05 57.425) (width 0.2) (layer "F.Cu") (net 10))
 (segment (start 147.949 56.599) (end 152.224 56.599) (width 0.2) (layer "F.Cu") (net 10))
 (segment (start 144 55.775) (end 144 55.3) (width 0.2) (layer "F.Cu") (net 6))
 (segment (start 145.55 57.325) (end 144 55.775) (width 0.2) (layer "F.Cu") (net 6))
 (segment (start 140.6 61.4) (end 141.25 60.75) (width 0.2) (layer "F.Cu") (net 6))
 (segment (start 141.25 60.75) (end 141.25 59.075) (width 0.2) (layer "F.Cu") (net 6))
 (via (at 140.6 61.4) (size 0.6) (drill 0.3) (layers "F.Cu" "B.Cu") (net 6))
 (via (at 144 55.3) (size 0.6) (drill 0.3) (layers "F.Cu" "B.Cu") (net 6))
 (segment (start 143.2 56.1) (end 143.2 61.4) (width 0.2) (layer "B.Cu") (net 6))
 (segment (start 143.2 61.4) (end 140.6 61.4) (width 0.2) (layer "B.Cu") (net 6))
 (segment (start 144 55.3) (end 143.2 56.1) (width 0.2) (layer "B.Cu") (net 6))
 (segment (start 149.252 51.8) (end 155.449 57.997) (width 0.2) (layer "F.Cu") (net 4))
 (segment (start 144.5 51.8) (end 149.252 51.8) (width 0.2) (layer "F.Cu") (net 4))
 (segment (start 155.449 63.674) (end 156.65 64.875) (width 0.2) (layer "F.Cu") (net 4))
 (segment (start 141.150057 51.8) (end 141.6 51.8) (width 0.2) (layer "F.Cu") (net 4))
 (segment (start 137.75 55.200057) (end 141.150057 51.8) (width 0.2) (layer "F.Cu") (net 4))
 (segment (start 137.75 57.325) (end 137.75 55.200057) (width 0.2) (layer "F.Cu") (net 4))
 (segment (start 155.449 57.997) (end 155.449 63.674) (width 0.2) (layer "F.Cu") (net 4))
 (via (at 144.5 51.8) (size 0.6) (drill 0.3) (layers "F.Cu" "B.Cu") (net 4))
 (via (at 141.6 51.8) (size 0.6) (drill 0.3) (layers "F.Cu" "B.Cu") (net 4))
 (segment (start 141.6 51.8) (end 144.5 51.8) (width 0.2) (layer "B.Cu") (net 4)))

